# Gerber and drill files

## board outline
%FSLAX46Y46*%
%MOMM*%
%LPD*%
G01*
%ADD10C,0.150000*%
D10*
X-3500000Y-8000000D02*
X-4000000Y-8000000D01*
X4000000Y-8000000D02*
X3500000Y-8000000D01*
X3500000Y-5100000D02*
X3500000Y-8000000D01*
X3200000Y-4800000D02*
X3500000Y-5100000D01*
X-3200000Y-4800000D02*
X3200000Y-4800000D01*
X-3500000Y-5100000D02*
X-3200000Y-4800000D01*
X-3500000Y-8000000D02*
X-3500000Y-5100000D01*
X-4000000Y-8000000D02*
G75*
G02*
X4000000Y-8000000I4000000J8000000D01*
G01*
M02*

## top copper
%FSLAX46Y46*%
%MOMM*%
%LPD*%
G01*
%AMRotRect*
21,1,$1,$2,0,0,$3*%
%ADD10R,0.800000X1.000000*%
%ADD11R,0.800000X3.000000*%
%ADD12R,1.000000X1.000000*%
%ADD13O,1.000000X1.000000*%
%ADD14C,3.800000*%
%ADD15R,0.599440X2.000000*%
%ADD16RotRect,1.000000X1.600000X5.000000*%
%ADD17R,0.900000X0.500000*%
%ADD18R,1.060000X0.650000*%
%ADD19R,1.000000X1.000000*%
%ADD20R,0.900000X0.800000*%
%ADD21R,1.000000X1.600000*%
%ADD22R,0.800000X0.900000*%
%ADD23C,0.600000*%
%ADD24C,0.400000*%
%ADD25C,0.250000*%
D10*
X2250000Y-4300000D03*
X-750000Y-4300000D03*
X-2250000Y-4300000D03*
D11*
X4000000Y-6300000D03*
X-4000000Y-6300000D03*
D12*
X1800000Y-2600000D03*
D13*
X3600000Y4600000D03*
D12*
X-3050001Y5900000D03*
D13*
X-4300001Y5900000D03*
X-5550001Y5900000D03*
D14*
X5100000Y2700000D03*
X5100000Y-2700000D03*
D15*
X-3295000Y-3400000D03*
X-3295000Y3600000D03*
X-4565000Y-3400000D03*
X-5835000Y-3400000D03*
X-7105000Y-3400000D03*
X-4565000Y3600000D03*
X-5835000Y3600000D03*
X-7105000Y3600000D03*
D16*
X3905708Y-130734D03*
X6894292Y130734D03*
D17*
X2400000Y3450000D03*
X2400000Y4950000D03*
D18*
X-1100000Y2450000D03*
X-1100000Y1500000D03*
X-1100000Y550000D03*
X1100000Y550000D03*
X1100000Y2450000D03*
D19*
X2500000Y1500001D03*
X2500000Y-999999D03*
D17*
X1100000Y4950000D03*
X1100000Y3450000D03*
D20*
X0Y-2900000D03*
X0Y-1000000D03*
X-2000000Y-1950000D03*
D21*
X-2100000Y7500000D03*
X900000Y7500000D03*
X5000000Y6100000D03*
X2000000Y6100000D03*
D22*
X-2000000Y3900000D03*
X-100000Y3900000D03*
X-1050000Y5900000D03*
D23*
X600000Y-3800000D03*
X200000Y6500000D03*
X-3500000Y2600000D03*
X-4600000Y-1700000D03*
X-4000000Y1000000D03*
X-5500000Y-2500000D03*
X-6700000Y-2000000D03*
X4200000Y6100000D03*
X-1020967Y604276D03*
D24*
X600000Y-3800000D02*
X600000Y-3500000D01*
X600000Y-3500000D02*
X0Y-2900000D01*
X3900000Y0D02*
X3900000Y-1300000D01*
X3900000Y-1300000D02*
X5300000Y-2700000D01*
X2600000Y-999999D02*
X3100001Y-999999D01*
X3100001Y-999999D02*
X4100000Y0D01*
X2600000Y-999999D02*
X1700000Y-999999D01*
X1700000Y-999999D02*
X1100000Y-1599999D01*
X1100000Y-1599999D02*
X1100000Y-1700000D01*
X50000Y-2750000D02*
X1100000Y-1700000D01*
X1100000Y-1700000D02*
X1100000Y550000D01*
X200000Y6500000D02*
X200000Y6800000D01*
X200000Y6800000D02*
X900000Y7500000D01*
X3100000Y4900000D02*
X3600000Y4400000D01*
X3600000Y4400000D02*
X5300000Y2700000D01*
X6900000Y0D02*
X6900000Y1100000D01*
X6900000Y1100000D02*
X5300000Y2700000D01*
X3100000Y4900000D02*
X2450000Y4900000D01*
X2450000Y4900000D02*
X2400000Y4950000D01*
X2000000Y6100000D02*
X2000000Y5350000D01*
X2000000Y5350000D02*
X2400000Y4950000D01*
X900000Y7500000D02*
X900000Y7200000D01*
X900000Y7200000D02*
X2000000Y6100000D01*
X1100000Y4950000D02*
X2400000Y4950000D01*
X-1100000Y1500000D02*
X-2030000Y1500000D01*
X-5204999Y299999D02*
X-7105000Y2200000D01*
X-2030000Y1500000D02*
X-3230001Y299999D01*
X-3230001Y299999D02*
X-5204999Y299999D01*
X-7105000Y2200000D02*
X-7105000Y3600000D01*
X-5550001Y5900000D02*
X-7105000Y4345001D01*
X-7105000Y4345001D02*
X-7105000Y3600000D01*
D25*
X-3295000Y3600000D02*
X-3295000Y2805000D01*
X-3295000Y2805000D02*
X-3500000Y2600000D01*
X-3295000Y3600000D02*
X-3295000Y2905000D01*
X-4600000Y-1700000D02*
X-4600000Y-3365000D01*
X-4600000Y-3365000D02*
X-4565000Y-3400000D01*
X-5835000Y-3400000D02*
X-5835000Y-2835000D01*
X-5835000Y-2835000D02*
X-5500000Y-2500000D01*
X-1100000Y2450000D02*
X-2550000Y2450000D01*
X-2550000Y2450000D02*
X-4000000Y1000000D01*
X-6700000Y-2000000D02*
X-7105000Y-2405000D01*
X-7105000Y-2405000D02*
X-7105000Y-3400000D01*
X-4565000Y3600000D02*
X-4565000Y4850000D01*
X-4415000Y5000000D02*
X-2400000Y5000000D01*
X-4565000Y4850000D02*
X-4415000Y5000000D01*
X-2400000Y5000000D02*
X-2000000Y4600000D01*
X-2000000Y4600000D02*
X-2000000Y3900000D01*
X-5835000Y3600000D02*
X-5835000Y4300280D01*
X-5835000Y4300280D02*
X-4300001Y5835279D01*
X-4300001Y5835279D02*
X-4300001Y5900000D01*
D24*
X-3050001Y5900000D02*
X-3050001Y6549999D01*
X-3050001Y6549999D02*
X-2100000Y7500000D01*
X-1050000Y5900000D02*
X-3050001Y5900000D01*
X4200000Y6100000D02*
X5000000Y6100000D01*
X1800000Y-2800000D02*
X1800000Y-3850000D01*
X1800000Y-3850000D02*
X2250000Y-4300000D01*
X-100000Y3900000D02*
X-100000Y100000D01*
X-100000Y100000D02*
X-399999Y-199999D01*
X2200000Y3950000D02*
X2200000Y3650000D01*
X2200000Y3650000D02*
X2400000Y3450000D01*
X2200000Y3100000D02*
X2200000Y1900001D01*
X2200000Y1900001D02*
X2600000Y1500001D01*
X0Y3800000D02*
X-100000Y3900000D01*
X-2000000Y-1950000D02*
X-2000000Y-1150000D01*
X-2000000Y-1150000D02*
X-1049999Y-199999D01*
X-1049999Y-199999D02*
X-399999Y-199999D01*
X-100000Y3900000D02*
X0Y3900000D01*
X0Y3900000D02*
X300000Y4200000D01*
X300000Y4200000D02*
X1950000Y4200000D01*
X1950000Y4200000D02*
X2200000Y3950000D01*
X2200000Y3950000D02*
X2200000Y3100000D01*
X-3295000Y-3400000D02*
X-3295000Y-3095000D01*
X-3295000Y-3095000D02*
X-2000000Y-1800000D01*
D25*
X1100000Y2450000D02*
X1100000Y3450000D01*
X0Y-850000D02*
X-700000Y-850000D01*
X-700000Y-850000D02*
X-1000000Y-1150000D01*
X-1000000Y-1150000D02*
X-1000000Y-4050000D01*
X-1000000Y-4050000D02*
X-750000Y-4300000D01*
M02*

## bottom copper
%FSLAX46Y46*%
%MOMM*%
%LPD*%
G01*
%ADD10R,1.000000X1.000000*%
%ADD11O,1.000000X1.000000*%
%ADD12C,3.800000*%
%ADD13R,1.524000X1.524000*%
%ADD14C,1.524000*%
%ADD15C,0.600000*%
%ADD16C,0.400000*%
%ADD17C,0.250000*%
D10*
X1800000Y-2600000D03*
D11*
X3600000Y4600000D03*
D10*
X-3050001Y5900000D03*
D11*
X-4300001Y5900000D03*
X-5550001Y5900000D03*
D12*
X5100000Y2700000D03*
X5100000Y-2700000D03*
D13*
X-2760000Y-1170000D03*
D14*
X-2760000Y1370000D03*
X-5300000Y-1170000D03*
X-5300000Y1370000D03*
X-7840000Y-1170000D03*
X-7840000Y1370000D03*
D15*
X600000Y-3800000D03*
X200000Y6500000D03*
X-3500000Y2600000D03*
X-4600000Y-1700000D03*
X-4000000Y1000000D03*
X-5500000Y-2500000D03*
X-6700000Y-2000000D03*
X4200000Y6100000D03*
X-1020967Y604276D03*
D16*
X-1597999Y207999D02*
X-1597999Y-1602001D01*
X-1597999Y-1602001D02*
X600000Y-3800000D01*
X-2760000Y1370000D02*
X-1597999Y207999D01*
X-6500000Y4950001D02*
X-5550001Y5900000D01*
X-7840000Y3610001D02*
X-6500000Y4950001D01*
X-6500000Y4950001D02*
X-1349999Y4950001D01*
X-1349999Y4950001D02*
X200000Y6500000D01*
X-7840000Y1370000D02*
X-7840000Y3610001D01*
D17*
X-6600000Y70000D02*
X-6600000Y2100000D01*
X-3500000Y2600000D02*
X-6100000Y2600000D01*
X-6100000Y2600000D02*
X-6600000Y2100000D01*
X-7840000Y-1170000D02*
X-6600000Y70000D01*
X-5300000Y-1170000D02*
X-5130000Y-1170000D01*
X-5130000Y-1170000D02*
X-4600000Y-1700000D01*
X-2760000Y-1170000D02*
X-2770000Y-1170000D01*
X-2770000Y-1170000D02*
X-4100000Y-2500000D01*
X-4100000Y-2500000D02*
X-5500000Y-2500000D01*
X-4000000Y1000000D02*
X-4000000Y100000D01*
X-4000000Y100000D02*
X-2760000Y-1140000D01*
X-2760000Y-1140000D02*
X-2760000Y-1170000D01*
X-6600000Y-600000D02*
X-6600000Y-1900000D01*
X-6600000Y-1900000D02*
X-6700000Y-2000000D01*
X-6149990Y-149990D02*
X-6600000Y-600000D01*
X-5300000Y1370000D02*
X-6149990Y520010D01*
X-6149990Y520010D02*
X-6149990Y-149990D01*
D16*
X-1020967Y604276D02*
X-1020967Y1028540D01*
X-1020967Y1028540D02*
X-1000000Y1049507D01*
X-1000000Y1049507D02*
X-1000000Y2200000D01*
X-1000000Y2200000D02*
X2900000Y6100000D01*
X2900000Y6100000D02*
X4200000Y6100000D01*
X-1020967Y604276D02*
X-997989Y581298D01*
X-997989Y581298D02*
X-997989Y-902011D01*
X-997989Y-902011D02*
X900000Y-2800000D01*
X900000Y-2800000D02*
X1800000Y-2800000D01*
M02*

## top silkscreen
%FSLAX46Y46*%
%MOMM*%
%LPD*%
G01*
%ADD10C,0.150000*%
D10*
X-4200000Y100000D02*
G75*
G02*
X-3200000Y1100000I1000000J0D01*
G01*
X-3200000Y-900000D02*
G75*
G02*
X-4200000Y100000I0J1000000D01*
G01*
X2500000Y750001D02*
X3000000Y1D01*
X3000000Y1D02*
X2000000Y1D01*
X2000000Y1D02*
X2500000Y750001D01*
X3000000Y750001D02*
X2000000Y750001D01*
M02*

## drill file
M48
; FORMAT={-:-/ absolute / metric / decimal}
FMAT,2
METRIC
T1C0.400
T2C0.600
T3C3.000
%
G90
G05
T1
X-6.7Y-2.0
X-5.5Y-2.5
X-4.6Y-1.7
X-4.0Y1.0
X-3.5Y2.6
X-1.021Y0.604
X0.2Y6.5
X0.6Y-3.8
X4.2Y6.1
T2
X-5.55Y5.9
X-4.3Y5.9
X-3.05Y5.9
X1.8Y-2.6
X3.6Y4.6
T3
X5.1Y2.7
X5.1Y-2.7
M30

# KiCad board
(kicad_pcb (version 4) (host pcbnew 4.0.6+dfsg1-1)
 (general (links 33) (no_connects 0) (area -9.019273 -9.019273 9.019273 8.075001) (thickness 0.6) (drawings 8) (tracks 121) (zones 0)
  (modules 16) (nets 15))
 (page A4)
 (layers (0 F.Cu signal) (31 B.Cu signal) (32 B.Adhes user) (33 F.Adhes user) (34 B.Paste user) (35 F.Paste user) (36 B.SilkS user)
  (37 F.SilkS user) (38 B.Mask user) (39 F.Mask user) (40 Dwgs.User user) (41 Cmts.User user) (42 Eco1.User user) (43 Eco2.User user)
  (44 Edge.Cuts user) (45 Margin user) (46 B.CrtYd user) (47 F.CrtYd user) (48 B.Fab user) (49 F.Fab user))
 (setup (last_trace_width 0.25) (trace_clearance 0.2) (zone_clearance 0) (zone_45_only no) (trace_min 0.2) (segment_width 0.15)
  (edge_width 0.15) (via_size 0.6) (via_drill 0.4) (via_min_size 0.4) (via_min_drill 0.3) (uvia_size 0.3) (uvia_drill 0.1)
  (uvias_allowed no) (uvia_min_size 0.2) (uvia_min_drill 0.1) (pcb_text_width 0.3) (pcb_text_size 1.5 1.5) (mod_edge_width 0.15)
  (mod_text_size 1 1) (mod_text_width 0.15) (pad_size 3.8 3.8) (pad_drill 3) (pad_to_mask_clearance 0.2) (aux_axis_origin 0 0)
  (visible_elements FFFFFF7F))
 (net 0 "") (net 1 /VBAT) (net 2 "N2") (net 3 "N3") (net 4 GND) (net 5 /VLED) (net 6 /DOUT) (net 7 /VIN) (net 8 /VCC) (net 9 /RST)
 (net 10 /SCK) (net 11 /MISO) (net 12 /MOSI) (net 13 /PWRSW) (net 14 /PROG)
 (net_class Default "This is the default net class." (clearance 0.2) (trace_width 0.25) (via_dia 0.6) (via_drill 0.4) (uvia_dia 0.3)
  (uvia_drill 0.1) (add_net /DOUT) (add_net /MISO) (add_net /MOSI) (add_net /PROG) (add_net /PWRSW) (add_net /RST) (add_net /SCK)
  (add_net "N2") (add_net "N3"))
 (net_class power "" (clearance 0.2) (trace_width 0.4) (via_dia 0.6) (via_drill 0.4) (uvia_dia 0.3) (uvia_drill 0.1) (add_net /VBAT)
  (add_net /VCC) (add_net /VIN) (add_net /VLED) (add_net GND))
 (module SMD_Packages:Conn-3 (layer F.Cu) (at 0 4.8)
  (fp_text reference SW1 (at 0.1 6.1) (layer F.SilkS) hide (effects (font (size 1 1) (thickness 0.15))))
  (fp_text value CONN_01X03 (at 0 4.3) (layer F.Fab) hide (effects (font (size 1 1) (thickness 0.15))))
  (pad 3 smd rect (at 2.25 -0.5) (size 0.8 1) (layers F.Cu F.Paste F.Mask) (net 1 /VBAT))
  (pad 2 smd rect (at -0.75 -0.5) (size 0.8 1) (layers F.Cu F.Paste F.Mask) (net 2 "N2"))
  (pad 1 smd rect (at -2.25 -0.5) (size 0.8 1) (layers F.Cu F.Paste F.Mask) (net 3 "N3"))
  (pad "" smd rect (at 4 1.5) (size 0.8 3) (layers F.Cu F.Paste F.Mask))
  (pad "" smd rect (at -4 1.5) (size 0.8 3) (layers F.Cu F.Paste F.Mask)))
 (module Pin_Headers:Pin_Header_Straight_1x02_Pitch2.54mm (layer F.Cu) (at 1.8 2.6 90)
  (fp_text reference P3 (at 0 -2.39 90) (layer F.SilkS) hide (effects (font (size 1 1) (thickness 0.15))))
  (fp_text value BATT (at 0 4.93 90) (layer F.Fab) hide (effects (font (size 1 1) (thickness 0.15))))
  (pad 1 thru_hole rect (at 0 0 90) (size 1 1) (drill 0.6) (layers *.Cu *.Mask) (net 1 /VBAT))
  (pad 2 thru_hole oval (at 7.2 1.8 90) (size 1 1) (drill 0.6) (layers *.Cu *.Mask) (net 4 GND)))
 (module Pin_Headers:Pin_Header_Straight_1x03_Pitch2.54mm (layer F.Cu) (at -3.050001 -5.9 270)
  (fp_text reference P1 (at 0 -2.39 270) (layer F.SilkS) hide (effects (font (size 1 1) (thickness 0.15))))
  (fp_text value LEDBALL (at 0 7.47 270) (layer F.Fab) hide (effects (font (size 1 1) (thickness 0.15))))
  (pad 1 thru_hole rect (at 0 0 270) (size 1 1) (drill 0.6) (layers *.Cu *.Mask) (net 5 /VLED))
  (pad 2 thru_hole oval (at 0 1.25 270) (size 1 1) (drill 0.6) (layers *.Cu *.Mask) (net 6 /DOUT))
  (pad 3 thru_hole oval (at 0 2.5 270) (size 1 1) (drill 0.6) (layers *.Cu *.Mask) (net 4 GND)))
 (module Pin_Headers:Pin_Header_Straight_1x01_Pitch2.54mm (layer B.Cu) (at 5.1 -2.7)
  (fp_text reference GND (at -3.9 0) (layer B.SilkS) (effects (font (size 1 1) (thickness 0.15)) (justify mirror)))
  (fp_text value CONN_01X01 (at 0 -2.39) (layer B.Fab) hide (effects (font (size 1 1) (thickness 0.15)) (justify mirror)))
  (pad 1 thru_hole circle (at 0 0) (size 3.8 3.8) (drill 3) (layers *.Cu *.Mask) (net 4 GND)))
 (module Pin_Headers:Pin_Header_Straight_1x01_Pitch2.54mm (layer B.Cu) (at 5.1 2.7 180)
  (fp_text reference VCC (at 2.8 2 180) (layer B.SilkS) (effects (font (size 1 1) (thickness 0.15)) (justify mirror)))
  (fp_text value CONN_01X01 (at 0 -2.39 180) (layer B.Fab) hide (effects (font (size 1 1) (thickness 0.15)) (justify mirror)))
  (pad 1 thru_hole circle (at 0 0 180) (size 3.8 3.8) (drill 3) (layers *.Cu *.Mask) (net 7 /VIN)))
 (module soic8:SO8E (layer F.Cu) (at -5.2 -0.1 180)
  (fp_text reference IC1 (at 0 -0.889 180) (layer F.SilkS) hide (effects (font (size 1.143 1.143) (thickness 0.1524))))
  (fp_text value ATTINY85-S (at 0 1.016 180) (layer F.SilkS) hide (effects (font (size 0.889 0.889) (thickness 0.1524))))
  (fp_arc (start -2 0) (end -1 0) (angle 90) (layer F.SilkS) (width 0.15))
  (fp_arc (start -2 0) (end -2 -1) (angle 90) (layer F.SilkS) (width 0.15))
  (pad 8 smd rect (at -1.905 -3.5 180) (size 0.59944 2) (layers F.Cu F.Paste F.Mask) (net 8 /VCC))
  (pad 1 smd rect (at -1.905 3.5 180) (size 0.59944 2) (layers F.Cu F.Paste F.Mask) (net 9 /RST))
  (pad 7 smd rect (at -0.635 -3.5 180) (size 0.59944 2) (layers F.Cu F.Paste F.Mask) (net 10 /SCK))
  (pad 6 smd rect (at 0.635 -3.5 180) (size 0.59944 2) (layers F.Cu F.Paste F.Mask) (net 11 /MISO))
  (pad 5 smd rect (at 1.905 -3.5 180) (size 0.59944 2) (layers F.Cu F.Paste F.Mask) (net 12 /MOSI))
  (pad 2 smd rect (at -0.635 3.5 180) (size 0.59944 2) (layers F.Cu F.Paste F.Mask) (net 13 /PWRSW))
  (pad 3 smd rect (at 0.635 3.5 180) (size 0.59944 2) (layers F.Cu F.Paste F.Mask) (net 6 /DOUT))
  (pad 4 smd rect (at 1.905 3.5 180) (size 0.59944 2) (layers F.Cu F.Paste F.Mask) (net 4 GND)))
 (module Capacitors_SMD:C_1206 (layer F.Cu) (at 5.4 0 5)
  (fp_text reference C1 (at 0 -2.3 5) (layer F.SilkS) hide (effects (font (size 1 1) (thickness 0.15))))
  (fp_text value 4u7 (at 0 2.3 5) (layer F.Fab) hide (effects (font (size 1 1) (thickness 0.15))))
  (pad 1 smd rect (at -1.5 0 5) (size 1 1.6) (layers F.Cu F.Paste F.Mask) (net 7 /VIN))
  (pad 2 smd rect (at 1.5 0 5) (size 1 1.6) (layers F.Cu F.Paste F.Mask) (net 4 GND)))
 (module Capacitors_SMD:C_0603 (layer F.Cu) (at 2.4 -4.2 90)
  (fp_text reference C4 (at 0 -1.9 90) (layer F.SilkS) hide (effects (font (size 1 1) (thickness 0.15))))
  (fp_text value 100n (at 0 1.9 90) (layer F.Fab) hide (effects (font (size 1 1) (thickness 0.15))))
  (pad 1 smd rect (at -0.75 0 90) (size 0.5 0.9) (layers F.Cu F.Paste F.Mask) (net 8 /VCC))
  (pad 2 smd rect (at 0.75 0 90) (size 0.5 0.9) (layers F.Cu F.Paste F.Mask) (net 4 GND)))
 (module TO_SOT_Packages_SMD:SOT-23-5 (layer F.Cu) (at 0 -1.5)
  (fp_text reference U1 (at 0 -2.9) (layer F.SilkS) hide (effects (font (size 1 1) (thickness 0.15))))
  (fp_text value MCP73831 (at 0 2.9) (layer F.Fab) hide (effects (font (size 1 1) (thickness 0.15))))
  (pad 1 smd rect (at -1.1 -0.95) (size 1.06 0.65) (layers F.Cu F.Paste F.Mask) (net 11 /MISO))
  (pad 2 smd rect (at -1.1 0) (size 1.06 0.65) (layers F.Cu F.Paste F.Mask) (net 4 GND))
  (pad 3 smd rect (at -1.1 0.95) (size 1.06 0.65) (layers F.Cu F.Paste F.Mask) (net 1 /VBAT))
  (pad 4 smd rect (at 1.1 0.95) (size 1.06 0.65) (layers F.Cu F.Paste F.Mask) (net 7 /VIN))
  (pad 5 smd rect (at 1.1 -0.95) (size 1.06 0.65) (layers F.Cu F.Paste F.Mask) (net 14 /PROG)))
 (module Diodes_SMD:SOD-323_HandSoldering (layer F.Cu) (at 2.5 -0.250001 270)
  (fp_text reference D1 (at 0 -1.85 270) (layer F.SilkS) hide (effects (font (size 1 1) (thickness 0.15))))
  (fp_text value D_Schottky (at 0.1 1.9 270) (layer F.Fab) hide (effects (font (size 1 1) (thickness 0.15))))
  (fp_line (start -0.5 0) (end 0.25 -0.5) (layer F.SilkS) (width 0.15))
  (fp_line (start 0.25 -0.5) (end 0.25 0.5) (layer F.SilkS) (width 0.15))
  (fp_line (start 0.25 0.5) (end -0.5 0) (layer F.SilkS) (width 0.15))
  (fp_line (start -0.5 -0.5) (end -0.5 0.5) (layer F.SilkS) (width 0.15))
  (pad 1 smd rect (at -1.25 0 270) (size 1 1) (layers F.Cu F.Paste F.Mask) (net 8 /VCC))
  (pad 2 smd rect (at 1.25 0 270) (size 1 1) (layers F.Cu F.Paste F.Mask) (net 7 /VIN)))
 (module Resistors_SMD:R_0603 (layer F.Cu) (at 1.1 -4.2 270)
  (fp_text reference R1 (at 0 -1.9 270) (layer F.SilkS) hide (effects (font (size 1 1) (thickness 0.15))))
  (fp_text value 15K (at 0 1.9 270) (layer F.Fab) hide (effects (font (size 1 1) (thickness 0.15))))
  (pad 1 smd rect (at -0.75 0 270) (size 0.5 0.9) (layers F.Cu F.Paste F.Mask) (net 4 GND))
  (pad 2 smd rect (at 0.75 0 270) (size 0.5 0.9) (layers F.Cu F.Paste F.Mask) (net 14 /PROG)))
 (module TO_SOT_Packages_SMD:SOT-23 (layer F.Cu) (at -1 1.95 180)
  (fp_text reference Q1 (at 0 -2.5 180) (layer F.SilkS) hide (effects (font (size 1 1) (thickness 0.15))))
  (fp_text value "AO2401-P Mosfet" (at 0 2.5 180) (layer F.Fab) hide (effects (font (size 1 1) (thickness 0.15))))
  (pad 1 smd rect (at -1 -0.95 180) (size 0.9 0.8) (layers F.Cu F.Paste F.Mask) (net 7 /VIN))
  (pad 2 smd rect (at -1 0.95 180) (size 0.9 0.8) (layers F.Cu F.Paste F.Mask) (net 2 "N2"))
  (pad 3 smd rect (at 1 0 180) (size 0.9 0.8) (layers F.Cu F.Paste F.Mask) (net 8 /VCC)))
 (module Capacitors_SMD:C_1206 (layer F.Cu) (at -0.6 -7.5)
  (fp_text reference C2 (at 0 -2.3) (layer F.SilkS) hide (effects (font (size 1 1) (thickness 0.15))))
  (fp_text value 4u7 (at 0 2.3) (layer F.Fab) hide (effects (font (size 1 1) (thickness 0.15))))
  (pad 1 smd rect (at -1.5 0) (size 1 1.6) (layers F.Cu F.Paste F.Mask) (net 5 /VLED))
  (pad 2 smd rect (at 1.5 0) (size 1 1.6) (layers F.Cu F.Paste F.Mask) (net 4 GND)))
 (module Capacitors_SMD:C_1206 (layer F.Cu) (at 3.5 -6.1 180)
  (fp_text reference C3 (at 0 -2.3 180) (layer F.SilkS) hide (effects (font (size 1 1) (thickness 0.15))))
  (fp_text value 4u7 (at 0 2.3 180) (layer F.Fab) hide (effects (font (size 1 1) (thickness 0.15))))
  (pad 1 smd rect (at -1.5 0 180) (size 1 1.6) (layers F.Cu F.Paste F.Mask) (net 1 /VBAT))
  (pad 2 smd rect (at 1.5 0 180) (size 1 1.6) (layers F.Cu F.Paste F.Mask) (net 4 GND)))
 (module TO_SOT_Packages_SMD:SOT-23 (layer F.Cu) (at -1.05 -4.9 90)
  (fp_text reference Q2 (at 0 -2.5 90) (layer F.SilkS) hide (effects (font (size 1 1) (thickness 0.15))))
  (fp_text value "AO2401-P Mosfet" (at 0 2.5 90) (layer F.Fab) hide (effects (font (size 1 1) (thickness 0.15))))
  (pad 1 smd rect (at -1 -0.95 90) (size 0.9 0.8) (layers F.Cu F.Paste F.Mask) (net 13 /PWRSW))
  (pad 2 smd rect (at -1 0.95 90) (size 0.9 0.8) (layers F.Cu F.Paste F.Mask) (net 8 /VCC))
  (pad 3 smd rect (at 1 0 90) (size 0.9 0.8) (layers F.Cu F.Paste F.Mask) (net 5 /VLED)))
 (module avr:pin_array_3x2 (layer B.Cu) (at -5.3 -0.1 180)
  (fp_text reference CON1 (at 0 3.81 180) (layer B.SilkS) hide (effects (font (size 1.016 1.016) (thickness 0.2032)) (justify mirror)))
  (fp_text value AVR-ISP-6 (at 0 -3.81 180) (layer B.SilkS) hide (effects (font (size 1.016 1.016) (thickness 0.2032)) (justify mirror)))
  (pad 1 smd rect (at -2.54 -1.27 180) (size 1.524 1.524) (layers B.Cu B.Paste B.Mask) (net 11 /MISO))
  (pad 2 smd circle (at -2.54 1.27 180) (size 1.524 1.524) (layers B.Cu B.Paste B.Mask) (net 7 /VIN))
  (pad 3 smd circle (at 0 -1.27 180) (size 1.524 1.524) (layers B.Cu B.Paste B.Mask) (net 10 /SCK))
  (pad 4 smd circle (at 0 1.27 180) (size 1.524 1.524) (layers B.Cu B.Paste B.Mask) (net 12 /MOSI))
  (pad 5 smd circle (at 2.54 -1.27 180) (size 1.524 1.524) (layers B.Cu B.Paste B.Mask) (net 9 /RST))
  (pad 6 smd circle (at 2.54 1.27 180) (size 1.524 1.524) (layers B.Cu B.Paste B.Mask) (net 4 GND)))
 (gr_line (start -3.5 8) (end -4 8) (layer Edge.Cuts) (width 0.15))
 (gr_line (start 4 8) (end 3.5 8) (layer Edge.Cuts) (width 0.15))
 (gr_line (start 3.5 5.1) (end 3.5 8) (angle 90) (layer Edge.Cuts) (width 0.15))
 (gr_line (start 3.2 4.8) (end 3.5 5.1) (angle 90) (layer Edge.Cuts) (width 0.15))
 (gr_line (start -3.2 4.8) (end 3.2 4.8) (angle 90) (layer Edge.Cuts) (width 0.15))
 (gr_line (start -3.5 5.1) (end -3.2 4.8) (angle 90) (layer Edge.Cuts) (width 0.15))
 (gr_line (start -3.5 8) (end -3.5 5.1) (angle 90) (layer Edge.Cuts) (width 0.15))
 (gr_arc (start 0 0) (end -4 8) (angle 306.8699005) (layer Edge.Cuts) (width 0.15))
 (segment (start 0.6 3.8) (end 0.6 3.5) (width 0.4) (layer F.Cu) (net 7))
 (segment (start 0.6 3.5) (end 0 2.9) (width 0.4) (layer F.Cu) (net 7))
 (segment (start -1.597999 -0.207999) (end -1.597999 1.602001) (width 0.4) (layer B.Cu) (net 7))
 (segment (start -1.597999 1.602001) (end 0.6 3.8) (width 0.4) (layer B.Cu) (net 7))
 (via (at 0.6 3.8) (size 0.6) (drill 0.4) (layers F.Cu B.Cu) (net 7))
 (segment (start 3.9 0) (end 3.9 1.3) (width 0.4) (layer F.Cu) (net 7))
 (segment (start 3.9 1.3) (end 5.3 2.7) (width 0.4) (layer F.Cu) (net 7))
 (segment (start -2.76 -1.37) (end -1.597999 -0.207999) (width 0.4) (layer B.Cu) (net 7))
 (segment (start 2.6 0.999999) (end 3.100001 0.999999) (width 0.4) (layer F.Cu) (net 7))
 (segment (start 3.100001 0.999999) (end 4.1 0) (width 0.4) (layer F.Cu) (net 7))
 (segment (start 2.6 0.999999) (end 1.7 0.999999) (width 0.4) (layer F.Cu) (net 7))
 (segment (start 1.7 0.999999) (end 1.1 1.599999) (width 0.4) (layer F.Cu) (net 7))
 (segment (start 1.1 1.599999) (end 1.1 1.7) (width 0.4) (layer F.Cu) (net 7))
 (segment (start 0.05 2.75) (end 1.1 1.7) (width 0.4) (layer F.Cu) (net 7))
 (segment (start 1.1 1.7) (end 1.1 -0.55) (width 0.4) (layer F.Cu) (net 7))
 (segment (start 0.2 -6.5) (end 0.2 -6.8) (width 0.4) (layer F.Cu) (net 4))
 (segment (start 0.2 -6.8) (end 0.9 -7.5) (width 0.4) (layer F.Cu) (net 4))
 (segment (start -6.5 -4.950001) (end -5.550001 -5.9) (width 0.4) (layer B.Cu) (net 4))
 (segment (start -7.84 -3.610001) (end -6.5 -4.950001) (width 0.4) (layer B.Cu) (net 4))
 (segment (start -6.5 -4.950001) (end -1.349999 -4.950001) (width 0.4) (layer B.Cu) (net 4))
 (via (at 0.2 -6.5) (size 0.6) (drill 0.4) (layers F.Cu B.Cu) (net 4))
 (segment (start -1.349999 -4.950001) (end 0.2 -6.5) (width 0.4) (layer B.Cu) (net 4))
 (segment (start 3.1 -4.9) (end 3.6 -4.4) (width 0.4) (layer F.Cu) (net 4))
 (segment (start 3.6 -4.4) (end 5.3 -2.7) (width 0.4) (layer F.Cu) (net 4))
 (segment (start 6.9 0) (end 6.9 -1.1) (width 0.4) (layer F.Cu) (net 4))
 (segment (start 6.9 -1.1) (end 5.3 -2.7) (width 0.4) (layer F.Cu) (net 4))
 (segment (start 3.1 -4.9) (end 2.45 -4.9) (width 0.4) (layer F.Cu) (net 4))
 (segment (start 2.45 -4.9) (end 2.4 -4.95) (width 0.4) (layer F.Cu) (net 4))
 (segment (start 2 -6.1) (end 2 -5.35) (width 0.4) (layer F.Cu) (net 4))
 (segment (start 2 -5.35) (end 2.4 -4.95) (width 0.4) (layer F.Cu) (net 4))
 (segment (start 0.9 -7.5) (end 0.9 -7.2) (width 0.4) (layer F.Cu) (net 4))
 (segment (start 0.9 -7.2) (end 2 -6.1) (width 0.4) (layer F.Cu) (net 4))
 (segment (start 1.1 -4.95) (end 2.4 -4.95) (width 0.4) (layer F.Cu) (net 4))
 (segment (start -1.1 -1.5) (end -2.03 -1.5) (width 0.4) (layer F.Cu) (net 4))
 (segment (start -5.204999 -0.299999) (end -7.105 -2.2) (width 0.4) (layer F.Cu) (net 4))
 (segment (start -2.03 -1.5) (end -3.230001 -0.299999) (width 0.4) (layer F.Cu) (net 4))
 (segment (start -3.230001 -0.299999) (end -5.204999 -0.299999) (width 0.4) (layer F.Cu) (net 4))
 (segment (start -7.105 -2.2) (end -7.105 -3.6) (width 0.4) (layer F.Cu) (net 4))
 (segment (start -7.84 -1.37) (end -7.84 -3.610001) (width 0.4) (layer B.Cu) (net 4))
 (segment (start -5.550001 -5.9) (end -7.105 -4.345001) (width 0.4) (layer F.Cu) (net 4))
 (segment (start -7.105 -4.345001) (end -7.105 -3.6) (width 0.4) (layer F.Cu) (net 4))
 (segment (start -6.6 -0.07) (end -6.6 -2.1) (width 0.25) (layer B.Cu) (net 9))
 (segment (start -3.5 -2.6) (end -6.1 -2.6) (width 0.25) (layer B.Cu) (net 9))
 (segment (start -6.1 -2.6) (end -6.6 -2.1) (width 0.25) (layer B.Cu) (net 9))
 (segment (start -3.295 -3.6) (end -3.295 -2.805) (width 0.25) (layer F.Cu) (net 9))
 (segment (start -3.295 -2.805) (end -3.5 -2.6) (width 0.25) (layer F.Cu) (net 9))
 (via (at -3.5 -2.6) (size 0.6) (drill 0.4) (layers F.Cu B.Cu) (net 9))
 (segment (start -3.295 -3.6) (end -3.295 -2.905) (width 0.25) (layer F.Cu) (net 9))
 (segment (start -7.84 1.17) (end -6.6 -0.07) (width 0.25) (layer B.Cu) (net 9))
 (segment (start -4.6 1.7) (end -4.6 3.365) (width 0.25) (layer F.Cu) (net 10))
 (segment (start -4.6 3.365) (end -4.565 3.4) (width 0.25) (layer F.Cu) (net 10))
 (segment (start -5.3 1.17) (end -5.13 1.17) (width 0.25) (layer B.Cu) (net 10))
 (segment (start -5.13 1.17) (end -4.6 1.7) (width 0.25) (layer B.Cu) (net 10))
 (via (at -4.6 1.7) (size 0.6) (drill 0.4) (layers F.Cu B.Cu) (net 10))
 (segment (start -2.76 1.17) (end -2.77 1.17) (width 0.25) (layer B.Cu) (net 11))
 (segment (start -2.77 1.17) (end -4.1 2.5) (width 0.25) (layer B.Cu) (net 11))
 (segment (start -4.1 2.5) (end -5.5 2.5) (width 0.25) (layer B.Cu) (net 11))
 (segment (start -4 -1) (end -4 -0.1) (width 0.25) (layer B.Cu) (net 11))
 (segment (start -4 -0.1) (end -2.76 1.14) (width 0.25) (layer B.Cu) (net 11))
 (segment (start -2.76 1.14) (end -2.76 1.17) (width 0.25) (layer B.Cu) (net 11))
 (segment (start -5.835 3.4) (end -5.835 2.835) (width 0.25) (layer F.Cu) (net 11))
 (segment (start -5.835 2.835) (end -5.5 2.5) (width 0.25) (layer F.Cu) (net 11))
 (segment (start -1.1 -2.45) (end -2.55 -2.45) (width 0.25) (layer F.Cu) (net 11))
 (segment (start -2.55 -2.45) (end -4 -1) (width 0.25) (layer F.Cu) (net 11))
 (via (at -4 -1) (size 0.6) (drill 0.4) (layers F.Cu B.Cu) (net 11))
 (via (at -5.5 2.5) (size 0.6) (drill 0.4) (layers F.Cu B.Cu) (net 11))
 (segment (start -6.7 2) (end -7.105 2.405) (width 0.25) (layer F.Cu) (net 12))
 (segment (start -7.105 2.405) (end -7.105 3.4) (width 0.25) (layer F.Cu) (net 12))
 (segment (start -6.6 0.6) (end -6.6 1.9) (width 0.25) (layer B.Cu) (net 12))
 (segment (start -6.6 1.9) (end -6.7 2) (width 0.25) (layer B.Cu) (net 12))
 (via (at -6.7 2) (size 0.6) (drill 0.4) (layers F.Cu B.Cu) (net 12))
 (segment (start -6.14999 0.14999) (end -6.6 0.6) (width 0.25) (layer B.Cu) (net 12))
 (segment (start -5.3 -1.37) (end -6.14999 -0.52001) (width 0.25) (layer B.Cu) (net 12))
 (segment (start -6.14999 -0.52001) (end -6.14999 0.14999) (width 0.25) (layer B.Cu) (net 12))
 (segment (start -4.565 -3.6) (end -4.565 -4.85) (width 0.25) (layer F.Cu) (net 13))
 (segment (start -4.415 -5) (end -2.4 -5) (width 0.25) (layer F.Cu) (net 13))
 (segment (start -4.565 -4.85) (end -4.415 -5) (width 0.25) (layer F.Cu) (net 13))
 (segment (start -2.4 -5) (end -2 -4.6) (width 0.25) (layer F.Cu) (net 13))
 (segment (start -2 -4.6) (end -2 -3.9) (width 0.25) (layer F.Cu) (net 13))
 (segment (start -5.835 -3.6) (end -5.835 -4.30028) (width 0.25) (layer F.Cu) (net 6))
 (segment (start -5.835 -4.30028) (end -4.300001 -5.835279) (width 0.25) (layer F.Cu) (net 6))
 (segment (start -4.300001 -5.835279) (end -4.300001 -5.9) (width 0.25) (layer F.Cu) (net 6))
 (segment (start -3.050001 -5.9) (end -3.050001 -6.549999) (width 0.4) (layer F.Cu) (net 5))
 (segment (start -3.050001 -6.549999) (end -2.1 -7.5) (width 0.4) (layer F.Cu) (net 5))
 (segment (start -1.05 -5.9) (end -3.050001 -5.9) (width 0.4) (layer F.Cu) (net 5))
 (segment (start -1.020967 -0.604276) (end -1.020967 -1.02854) (width 0.4) (layer B.Cu) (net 1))
 (segment (start -1.020967 -1.02854) (end -1 -1.049507) (width 0.4) (layer B.Cu) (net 1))
 (segment (start -1 -1.049507) (end -1 -2.2) (width 0.4) (layer B.Cu) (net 1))
 (segment (start -1 -2.2) (end 2.9 -6.1) (width 0.4) (layer B.Cu) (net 1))
 (segment (start 2.9 -6.1) (end 4.2 -6.1) (width 0.4) (layer B.Cu) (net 1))
 (segment (start 4.2 -6.1) (end 5 -6.1) (width 0.4) (layer F.Cu) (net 1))
 (via (at 4.2 -6.1) (size 0.6) (drill 0.4) (layers F.Cu B.Cu) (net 1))
 (segment (start -1.020967 -0.604276) (end -0.997989 -0.581298) (width 0.4) (layer B.Cu) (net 1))
 (segment (start -0.997989 -0.581298) (end -0.997989 0.902011) (width 0.4) (layer B.Cu) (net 1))
 (segment (start -0.997989 0.902011) (end 0.9 2.8) (width 0.4) (layer B.Cu) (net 1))
 (segment (start 0.9 2.8) (end 1.8 2.8) (width 0.4) (layer B.Cu) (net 1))
 (segment (start 1.8 2.8) (end 1.8 3.85) (width 0.4) (layer F.Cu) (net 1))
 (segment (start 1.8 3.85) (end 2.25 4.3) (width 0.4) (layer F.Cu) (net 1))
 (via (at -1.020967 -0.604276) (size 0.6) (drill 0.4) (layers F.Cu B.Cu) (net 1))
 (segment (start -0.1 -3.9) (end -0.1 -0.1) (width 0.4) (layer F.Cu) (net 8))
 (segment (start -0.1 -0.1) (end -0.399999 0.199999) (width 0.4) (layer F.Cu) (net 8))
 (segment (start 2.2 -3.95) (end 2.2 -3.65) (width 0.4) (layer F.Cu) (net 8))
 (segment (start 2.2 -3.65) (end 2.4 -3.45) (width 0.4) (layer F.Cu) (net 8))
 (segment (start 2.2 -3.1) (end 2.2 -1.900001) (width 0.4) (layer F.Cu) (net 8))
 (segment (start 2.2 -1.900001) (end 2.6 -1.500001) (width 0.4) (layer F.Cu) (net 8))
 (segment (start 0 -3.8) (end -0.1 -3.9) (width 0.4) (layer F.Cu) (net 8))
 (segment (start -2 1.95) (end -2 1.15) (width 0.4) (layer F.Cu) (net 8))
 (segment (start -2 1.15) (end -1.049999 0.199999) (width 0.4) (layer F.Cu) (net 8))
 (segment (start -1.049999 0.199999) (end -0.399999 0.199999) (width 0.4) (layer F.Cu) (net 8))
 (segment (start -0.1 -3.9) (end 0 -3.9) (width 0.4) (layer F.Cu) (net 8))
 (segment (start 0 -3.9) (end 0.3 -4.2) (width 0.4) (layer F.Cu) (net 8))
 (segment (start 0.3 -4.2) (end 1.95 -4.2) (width 0.4) (layer F.Cu) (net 8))
 (segment (start 1.95 -4.2) (end 2.2 -3.95) (width 0.4) (layer F.Cu) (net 8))
 (segment (start 2.2 -3.95) (end 2.2 -3.1) (width 0.4) (layer F.Cu) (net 8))
 (segment (start -3.295 3.4) (end -3.295 3.095) (width 0.4) (layer F.Cu) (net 8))
 (segment (start -3.295 3.095) (end -2 1.8) (width 0.4) (layer F.Cu) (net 8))
 (segment (start 1.1 -2.45) (end 1.1 -3.45) (width 0.25) (layer F.Cu) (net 14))
 (segment (start 0 0.85) (end -0.7 0.85) (width 0.25) (layer F.Cu) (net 2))
 (segment (start -0.7 0.85) (end -1 1.15) (width 0.25) (layer F.Cu) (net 2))
 (segment (start -1 1.15) (end -1 4.05) (width 0.25) (layer F.Cu) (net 2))
 (segment (start -1 4.05) (end -0.75 4.3) (width 0.25) (layer F.Cu) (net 2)))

